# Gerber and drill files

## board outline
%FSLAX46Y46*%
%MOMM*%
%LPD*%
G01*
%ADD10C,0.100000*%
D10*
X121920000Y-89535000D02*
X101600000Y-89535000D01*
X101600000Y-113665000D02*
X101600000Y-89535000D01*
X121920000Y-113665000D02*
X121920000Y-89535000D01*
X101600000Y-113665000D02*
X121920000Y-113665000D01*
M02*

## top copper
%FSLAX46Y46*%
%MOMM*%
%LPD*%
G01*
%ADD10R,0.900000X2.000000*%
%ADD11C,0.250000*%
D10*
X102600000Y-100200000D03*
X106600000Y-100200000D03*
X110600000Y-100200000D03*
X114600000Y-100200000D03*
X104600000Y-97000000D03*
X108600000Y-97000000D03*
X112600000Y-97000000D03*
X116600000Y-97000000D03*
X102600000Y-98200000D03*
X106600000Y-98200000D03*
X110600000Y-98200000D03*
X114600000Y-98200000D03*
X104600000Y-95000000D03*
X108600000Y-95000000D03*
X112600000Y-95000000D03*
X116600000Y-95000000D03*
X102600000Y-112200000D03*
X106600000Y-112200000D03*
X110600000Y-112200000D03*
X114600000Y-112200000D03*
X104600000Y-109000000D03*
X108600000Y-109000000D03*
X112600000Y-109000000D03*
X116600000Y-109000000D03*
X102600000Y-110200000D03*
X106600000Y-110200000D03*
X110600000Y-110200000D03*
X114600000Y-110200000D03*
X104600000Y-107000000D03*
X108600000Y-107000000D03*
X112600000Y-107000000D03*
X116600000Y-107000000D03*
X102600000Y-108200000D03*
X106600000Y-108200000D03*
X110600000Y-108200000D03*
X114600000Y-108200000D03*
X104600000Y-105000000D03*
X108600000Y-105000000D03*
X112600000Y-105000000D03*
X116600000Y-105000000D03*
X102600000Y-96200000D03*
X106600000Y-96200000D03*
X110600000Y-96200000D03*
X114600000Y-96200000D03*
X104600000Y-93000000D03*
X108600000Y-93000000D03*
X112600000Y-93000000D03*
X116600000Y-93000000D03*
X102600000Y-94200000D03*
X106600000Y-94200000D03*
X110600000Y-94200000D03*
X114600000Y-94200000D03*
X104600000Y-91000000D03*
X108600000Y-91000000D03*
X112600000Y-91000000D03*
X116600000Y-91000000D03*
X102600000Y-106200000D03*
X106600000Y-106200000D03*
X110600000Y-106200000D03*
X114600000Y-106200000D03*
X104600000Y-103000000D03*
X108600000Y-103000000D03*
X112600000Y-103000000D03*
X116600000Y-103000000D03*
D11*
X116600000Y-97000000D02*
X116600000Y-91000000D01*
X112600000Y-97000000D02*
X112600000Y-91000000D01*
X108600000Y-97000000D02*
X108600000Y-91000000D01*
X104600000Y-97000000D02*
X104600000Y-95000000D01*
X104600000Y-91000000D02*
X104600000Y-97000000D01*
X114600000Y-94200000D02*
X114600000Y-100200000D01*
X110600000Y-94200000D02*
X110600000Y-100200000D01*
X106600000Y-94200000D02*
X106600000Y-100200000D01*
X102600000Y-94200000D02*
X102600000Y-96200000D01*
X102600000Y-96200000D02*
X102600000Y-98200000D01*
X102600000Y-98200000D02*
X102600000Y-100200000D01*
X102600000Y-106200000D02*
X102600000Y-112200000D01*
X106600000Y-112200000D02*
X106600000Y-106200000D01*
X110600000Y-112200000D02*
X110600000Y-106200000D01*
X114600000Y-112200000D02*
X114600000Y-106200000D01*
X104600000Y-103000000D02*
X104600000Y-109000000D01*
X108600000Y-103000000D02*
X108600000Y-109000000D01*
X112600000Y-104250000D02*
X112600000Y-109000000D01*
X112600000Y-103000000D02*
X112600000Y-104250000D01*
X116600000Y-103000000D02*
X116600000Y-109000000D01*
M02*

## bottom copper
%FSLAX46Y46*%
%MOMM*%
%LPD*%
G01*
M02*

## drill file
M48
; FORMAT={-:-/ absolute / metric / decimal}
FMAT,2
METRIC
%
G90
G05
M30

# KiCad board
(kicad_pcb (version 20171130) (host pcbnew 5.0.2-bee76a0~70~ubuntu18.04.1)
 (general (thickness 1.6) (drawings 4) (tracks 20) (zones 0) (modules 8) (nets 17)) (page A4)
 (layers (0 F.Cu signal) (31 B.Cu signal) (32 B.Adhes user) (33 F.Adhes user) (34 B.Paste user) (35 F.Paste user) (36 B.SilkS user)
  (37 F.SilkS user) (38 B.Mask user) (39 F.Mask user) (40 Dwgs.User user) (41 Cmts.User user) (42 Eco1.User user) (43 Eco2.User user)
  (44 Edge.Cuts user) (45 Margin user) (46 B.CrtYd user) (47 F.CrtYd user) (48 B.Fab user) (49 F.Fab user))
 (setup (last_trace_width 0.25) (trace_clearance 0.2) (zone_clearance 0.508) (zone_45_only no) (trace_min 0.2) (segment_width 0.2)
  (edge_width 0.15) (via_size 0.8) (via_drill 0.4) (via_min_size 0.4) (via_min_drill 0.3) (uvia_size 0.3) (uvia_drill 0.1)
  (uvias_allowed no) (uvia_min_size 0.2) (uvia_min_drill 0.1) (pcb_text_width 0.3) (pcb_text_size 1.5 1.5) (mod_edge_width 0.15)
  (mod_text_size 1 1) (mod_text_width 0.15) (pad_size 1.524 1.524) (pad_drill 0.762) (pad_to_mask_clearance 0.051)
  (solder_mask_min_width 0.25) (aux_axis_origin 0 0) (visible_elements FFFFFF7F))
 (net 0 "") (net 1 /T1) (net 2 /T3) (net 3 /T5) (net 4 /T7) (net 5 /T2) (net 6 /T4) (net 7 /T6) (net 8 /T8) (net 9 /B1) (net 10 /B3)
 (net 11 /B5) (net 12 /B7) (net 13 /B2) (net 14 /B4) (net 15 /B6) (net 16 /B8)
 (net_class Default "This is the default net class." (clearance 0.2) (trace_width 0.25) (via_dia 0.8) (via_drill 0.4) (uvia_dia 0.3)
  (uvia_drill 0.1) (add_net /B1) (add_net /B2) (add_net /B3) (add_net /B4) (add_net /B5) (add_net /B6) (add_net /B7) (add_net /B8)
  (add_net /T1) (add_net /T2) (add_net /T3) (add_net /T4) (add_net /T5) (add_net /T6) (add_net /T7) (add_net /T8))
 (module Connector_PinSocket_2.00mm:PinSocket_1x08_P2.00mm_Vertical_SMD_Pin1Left (layer F.Cu) (at 109.6 98.6 90)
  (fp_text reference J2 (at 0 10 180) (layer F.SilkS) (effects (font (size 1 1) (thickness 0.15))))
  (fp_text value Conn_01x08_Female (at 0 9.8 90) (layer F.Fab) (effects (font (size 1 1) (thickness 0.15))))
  (pad 1 smd rect (at -1.6 -7 90) (size 2 0.9) (layers F.Cu F.Paste F.Mask) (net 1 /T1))
  (pad 3 smd rect (at -1.6 -3 90) (size 2 0.9) (layers F.Cu F.Paste F.Mask) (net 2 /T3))
  (pad 5 smd rect (at -1.6 1 90) (size 2 0.9) (layers F.Cu F.Paste F.Mask) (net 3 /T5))
  (pad 7 smd rect (at -1.6 5 90) (size 2 0.9) (layers F.Cu F.Paste F.Mask) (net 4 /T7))
  (pad 2 smd rect (at 1.6 -5 90) (size 2 0.9) (layers F.Cu F.Paste F.Mask) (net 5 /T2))
  (pad 4 smd rect (at 1.6 -1 90) (size 2 0.9) (layers F.Cu F.Paste F.Mask) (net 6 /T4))
  (pad 6 smd rect (at 1.6 3 90) (size 2 0.9) (layers F.Cu F.Paste F.Mask) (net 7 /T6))
  (pad 8 smd rect (at 1.6 7 90) (size 2 0.9) (layers F.Cu F.Paste F.Mask) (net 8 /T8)))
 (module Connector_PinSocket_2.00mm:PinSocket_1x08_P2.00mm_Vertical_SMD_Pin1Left (layer F.Cu) (at 109.6 96.6 90)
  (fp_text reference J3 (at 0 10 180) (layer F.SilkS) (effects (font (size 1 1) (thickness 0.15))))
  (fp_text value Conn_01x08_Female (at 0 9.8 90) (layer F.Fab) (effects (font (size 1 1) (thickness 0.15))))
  (pad 1 smd rect (at -1.6 -7 90) (size 2 0.9) (layers F.Cu F.Paste F.Mask) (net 1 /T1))
  (pad 3 smd rect (at -1.6 -3 90) (size 2 0.9) (layers F.Cu F.Paste F.Mask) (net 2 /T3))
  (pad 5 smd rect (at -1.6 1 90) (size 2 0.9) (layers F.Cu F.Paste F.Mask) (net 3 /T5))
  (pad 7 smd rect (at -1.6 5 90) (size 2 0.9) (layers F.Cu F.Paste F.Mask) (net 4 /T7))
  (pad 2 smd rect (at 1.6 -5 90) (size 2 0.9) (layers F.Cu F.Paste F.Mask) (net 5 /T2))
  (pad 4 smd rect (at 1.6 -1 90) (size 2 0.9) (layers F.Cu F.Paste F.Mask) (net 6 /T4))
  (pad 6 smd rect (at 1.6 3 90) (size 2 0.9) (layers F.Cu F.Paste F.Mask) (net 7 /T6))
  (pad 8 smd rect (at 1.6 7 90) (size 2 0.9) (layers F.Cu F.Paste F.Mask) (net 8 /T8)))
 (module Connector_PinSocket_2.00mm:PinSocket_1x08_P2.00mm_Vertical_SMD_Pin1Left (layer F.Cu) (at 109.6 110.6 90)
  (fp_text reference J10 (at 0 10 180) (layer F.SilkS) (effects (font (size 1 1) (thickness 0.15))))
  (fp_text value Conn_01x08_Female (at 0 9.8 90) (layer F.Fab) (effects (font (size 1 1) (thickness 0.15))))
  (pad 1 smd rect (at -1.6 -7 90) (size 2 0.9) (layers F.Cu F.Paste F.Mask) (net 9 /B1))
  (pad 3 smd rect (at -1.6 -3 90) (size 2 0.9) (layers F.Cu F.Paste F.Mask) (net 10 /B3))
  (pad 5 smd rect (at -1.6 1 90) (size 2 0.9) (layers F.Cu F.Paste F.Mask) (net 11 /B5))
  (pad 7 smd rect (at -1.6 5 90) (size 2 0.9) (layers F.Cu F.Paste F.Mask) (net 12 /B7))
  (pad 2 smd rect (at 1.6 -5 90) (size 2 0.9) (layers F.Cu F.Paste F.Mask) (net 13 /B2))
  (pad 4 smd rect (at 1.6 -1 90) (size 2 0.9) (layers F.Cu F.Paste F.Mask) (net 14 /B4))
  (pad 6 smd rect (at 1.6 3 90) (size 2 0.9) (layers F.Cu F.Paste F.Mask) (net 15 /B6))
  (pad 8 smd rect (at 1.6 7 90) (size 2 0.9) (layers F.Cu F.Paste F.Mask) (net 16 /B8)))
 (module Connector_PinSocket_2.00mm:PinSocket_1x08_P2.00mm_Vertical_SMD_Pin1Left (layer F.Cu) (at 109.6 108.6 90)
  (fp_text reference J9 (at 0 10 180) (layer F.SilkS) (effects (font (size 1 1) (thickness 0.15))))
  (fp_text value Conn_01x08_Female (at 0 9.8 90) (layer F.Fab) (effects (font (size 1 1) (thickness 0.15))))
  (pad 1 smd rect (at -1.6 -7 90) (size 2 0.9) (layers F.Cu F.Paste F.Mask) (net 9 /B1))
  (pad 3 smd rect (at -1.6 -3 90) (size 2 0.9) (layers F.Cu F.Paste F.Mask) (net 10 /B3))
  (pad 5 smd rect (at -1.6 1 90) (size 2 0.9) (layers F.Cu F.Paste F.Mask) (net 11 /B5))
  (pad 7 smd rect (at -1.6 5 90) (size 2 0.9) (layers F.Cu F.Paste F.Mask) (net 12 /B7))
  (pad 2 smd rect (at 1.6 -5 90) (size 2 0.9) (layers F.Cu F.Paste F.Mask) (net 13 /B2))
  (pad 4 smd rect (at 1.6 -1 90) (size 2 0.9) (layers F.Cu F.Paste F.Mask) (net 14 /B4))
  (pad 6 smd rect (at 1.6 3 90) (size 2 0.9) (layers F.Cu F.Paste F.Mask) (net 15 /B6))
  (pad 8 smd rect (at 1.6 7 90) (size 2 0.9) (layers F.Cu F.Paste F.Mask) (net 16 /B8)))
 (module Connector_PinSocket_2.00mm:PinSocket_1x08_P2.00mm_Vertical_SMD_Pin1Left (layer F.Cu) (at 109.6 106.6 90)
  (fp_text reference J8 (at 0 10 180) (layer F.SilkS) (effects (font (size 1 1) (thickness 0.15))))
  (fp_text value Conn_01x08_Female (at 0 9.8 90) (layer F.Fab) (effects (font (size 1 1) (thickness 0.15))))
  (pad 1 smd rect (at -1.6 -7 90) (size 2 0.9) (layers F.Cu F.Paste F.Mask) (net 9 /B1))
  (pad 3 smd rect (at -1.6 -3 90) (size 2 0.9) (layers F.Cu F.Paste F.Mask) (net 10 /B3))
  (pad 5 smd rect (at -1.6 1 90) (size 2 0.9) (layers F.Cu F.Paste F.Mask) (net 11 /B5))
  (pad 7 smd rect (at -1.6 5 90) (size 2 0.9) (layers F.Cu F.Paste F.Mask) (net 12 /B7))
  (pad 2 smd rect (at 1.6 -5 90) (size 2 0.9) (layers F.Cu F.Paste F.Mask) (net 13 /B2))
  (pad 4 smd rect (at 1.6 -1 90) (size 2 0.9) (layers F.Cu F.Paste F.Mask) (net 14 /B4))
  (pad 6 smd rect (at 1.6 3 90) (size 2 0.9) (layers F.Cu F.Paste F.Mask) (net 15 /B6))
  (pad 8 smd rect (at 1.6 7 90) (size 2 0.9) (layers F.Cu F.Paste F.Mask) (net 16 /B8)))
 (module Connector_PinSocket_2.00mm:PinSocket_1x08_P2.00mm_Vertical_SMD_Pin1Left (layer F.Cu) (at 109.6 94.6 90)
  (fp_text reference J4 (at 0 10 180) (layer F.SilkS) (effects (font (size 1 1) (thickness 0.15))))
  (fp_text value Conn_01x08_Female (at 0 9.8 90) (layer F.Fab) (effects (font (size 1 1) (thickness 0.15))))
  (pad 1 smd rect (at -1.6 -7 90) (size 2 0.9) (layers F.Cu F.Paste F.Mask) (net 1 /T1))
  (pad 3 smd rect (at -1.6 -3 90) (size 2 0.9) (layers F.Cu F.Paste F.Mask) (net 2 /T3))
  (pad 5 smd rect (at -1.6 1 90) (size 2 0.9) (layers F.Cu F.Paste F.Mask) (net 3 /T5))
  (pad 7 smd rect (at -1.6 5 90) (size 2 0.9) (layers F.Cu F.Paste F.Mask) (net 4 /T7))
  (pad 2 smd rect (at 1.6 -5 90) (size 2 0.9) (layers F.Cu F.Paste F.Mask) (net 5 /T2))
  (pad 4 smd rect (at 1.6 -1 90) (size 2 0.9) (layers F.Cu F.Paste F.Mask) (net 6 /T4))
  (pad 6 smd rect (at 1.6 3 90) (size 2 0.9) (layers F.Cu F.Paste F.Mask) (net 7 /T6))
  (pad 8 smd rect (at 1.6 7 90) (size 2 0.9) (layers F.Cu F.Paste F.Mask) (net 8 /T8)))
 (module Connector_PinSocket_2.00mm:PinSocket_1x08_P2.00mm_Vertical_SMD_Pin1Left (layer F.Cu) (at 109.6 92.6 90)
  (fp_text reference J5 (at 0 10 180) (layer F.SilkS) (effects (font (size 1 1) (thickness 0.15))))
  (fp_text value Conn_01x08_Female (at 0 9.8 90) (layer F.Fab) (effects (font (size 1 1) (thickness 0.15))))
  (pad 1 smd rect (at -1.6 -7 90) (size 2 0.9) (layers F.Cu F.Paste F.Mask) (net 1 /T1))
  (pad 3 smd rect (at -1.6 -3 90) (size 2 0.9) (layers F.Cu F.Paste F.Mask) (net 2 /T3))
  (pad 5 smd rect (at -1.6 1 90) (size 2 0.9) (layers F.Cu F.Paste F.Mask) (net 3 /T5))
  (pad 7 smd rect (at -1.6 5 90) (size 2 0.9) (layers F.Cu F.Paste F.Mask) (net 4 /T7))
  (pad 2 smd rect (at 1.6 -5 90) (size 2 0.9) (layers F.Cu F.Paste F.Mask) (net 5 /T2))
  (pad 4 smd rect (at 1.6 -1 90) (size 2 0.9) (layers F.Cu F.Paste F.Mask) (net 6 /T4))
  (pad 6 smd rect (at 1.6 3 90) (size 2 0.9) (layers F.Cu F.Paste F.Mask) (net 7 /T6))
  (pad 8 smd rect (at 1.6 7 90) (size 2 0.9) (layers F.Cu F.Paste F.Mask) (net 8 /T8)))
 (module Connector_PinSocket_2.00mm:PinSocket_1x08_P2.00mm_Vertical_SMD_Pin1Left (layer F.Cu) (at 109.6 104.6 90)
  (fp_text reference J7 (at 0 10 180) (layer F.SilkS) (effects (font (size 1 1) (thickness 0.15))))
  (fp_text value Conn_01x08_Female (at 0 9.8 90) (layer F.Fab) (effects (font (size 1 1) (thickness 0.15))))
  (pad 1 smd rect (at -1.6 -7 90) (size 2 0.9) (layers F.Cu F.Paste F.Mask) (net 9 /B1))
  (pad 3 smd rect (at -1.6 -3 90) (size 2 0.9) (layers F.Cu F.Paste F.Mask) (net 10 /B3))
  (pad 5 smd rect (at -1.6 1 90) (size 2 0.9) (layers F.Cu F.Paste F.Mask) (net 11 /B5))
  (pad 7 smd rect (at -1.6 5 90) (size 2 0.9) (layers F.Cu F.Paste F.Mask) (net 12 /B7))
  (pad 2 smd rect (at 1.6 -5 90) (size 2 0.9) (layers F.Cu F.Paste F.Mask) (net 13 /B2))
  (pad 4 smd rect (at 1.6 -1 90) (size 2 0.9) (layers F.Cu F.Paste F.Mask) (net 14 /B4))
  (pad 6 smd rect (at 1.6 3 90) (size 2 0.9) (layers F.Cu F.Paste F.Mask) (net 15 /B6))
  (pad 8 smd rect (at 1.6 7 90) (size 2 0.9) (layers F.Cu F.Paste F.Mask) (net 16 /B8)))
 (gr_line (start 121.92 89.535) (end 101.6 89.535) (layer Edge.Cuts) (width 0.1))
 (gr_line (start 101.6 113.665) (end 101.6 89.535) (layer Edge.Cuts) (width 0.1))
 (gr_line (start 121.92 113.665) (end 121.92 89.535) (layer Edge.Cuts) (width 0.1))
 (gr_line (start 101.6 113.665) (end 121.92 113.665) (layer Edge.Cuts) (width 0.1))
 (segment (start 116.6 97) (end 116.6 91) (width 0.25) (layer F.Cu) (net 8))
 (segment (start 112.6 97) (end 112.6 91) (width 0.25) (layer F.Cu) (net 7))
 (segment (start 108.6 97) (end 108.6 91) (width 0.25) (layer F.Cu) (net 6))
 (segment (start 104.6 97) (end 104.6 95) (width 0.25) (layer F.Cu) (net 5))
 (segment (start 104.6 91) (end 104.6 97) (width 0.25) (layer F.Cu) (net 5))
 (segment (start 114.6 94.2) (end 114.6 100.2) (width 0.25) (layer F.Cu) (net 4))
 (segment (start 110.6 94.2) (end 110.6 100.2) (width 0.25) (layer F.Cu) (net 3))
 (segment (start 106.6 94.2) (end 106.6 100.2) (width 0.25) (layer F.Cu) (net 2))
 (segment (start 102.6 94.2) (end 102.6 96.2) (width 0.25) (layer F.Cu) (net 1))
 (segment (start 102.6 96.2) (end 102.6 98.2) (width 0.25) (layer F.Cu) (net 1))
 (segment (start 102.6 98.2) (end 102.6 100.2) (width 0.25) (layer F.Cu) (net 1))
 (segment (start 102.6 106.2) (end 102.6 112.2) (width 0.25) (layer F.Cu) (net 9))
 (segment (start 106.6 112.2) (end 106.6 106.2) (width 0.25) (layer F.Cu) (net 10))
 (segment (start 110.6 112.2) (end 110.6 106.2) (width 0.25) (layer F.Cu) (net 11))
 (segment (start 114.6 112.2) (end 114.6 106.2) (width 0.25) (layer F.Cu) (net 12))
 (segment (start 104.6 103) (end 104.6 109) (width 0.25) (layer F.Cu) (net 13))
 (segment (start 108.6 103) (end 108.6 109) (width 0.25) (layer F.Cu) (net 14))
 (segment (start 112.6 104.25) (end 112.6 109) (width 0.25) (layer F.Cu) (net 15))
 (segment (start 112.6 103) (end 112.6 104.25) (width 0.25) (layer F.Cu) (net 15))
 (segment (start 116.6 103) (end 116.6 109) (width 0.25) (layer F.Cu) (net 16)))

